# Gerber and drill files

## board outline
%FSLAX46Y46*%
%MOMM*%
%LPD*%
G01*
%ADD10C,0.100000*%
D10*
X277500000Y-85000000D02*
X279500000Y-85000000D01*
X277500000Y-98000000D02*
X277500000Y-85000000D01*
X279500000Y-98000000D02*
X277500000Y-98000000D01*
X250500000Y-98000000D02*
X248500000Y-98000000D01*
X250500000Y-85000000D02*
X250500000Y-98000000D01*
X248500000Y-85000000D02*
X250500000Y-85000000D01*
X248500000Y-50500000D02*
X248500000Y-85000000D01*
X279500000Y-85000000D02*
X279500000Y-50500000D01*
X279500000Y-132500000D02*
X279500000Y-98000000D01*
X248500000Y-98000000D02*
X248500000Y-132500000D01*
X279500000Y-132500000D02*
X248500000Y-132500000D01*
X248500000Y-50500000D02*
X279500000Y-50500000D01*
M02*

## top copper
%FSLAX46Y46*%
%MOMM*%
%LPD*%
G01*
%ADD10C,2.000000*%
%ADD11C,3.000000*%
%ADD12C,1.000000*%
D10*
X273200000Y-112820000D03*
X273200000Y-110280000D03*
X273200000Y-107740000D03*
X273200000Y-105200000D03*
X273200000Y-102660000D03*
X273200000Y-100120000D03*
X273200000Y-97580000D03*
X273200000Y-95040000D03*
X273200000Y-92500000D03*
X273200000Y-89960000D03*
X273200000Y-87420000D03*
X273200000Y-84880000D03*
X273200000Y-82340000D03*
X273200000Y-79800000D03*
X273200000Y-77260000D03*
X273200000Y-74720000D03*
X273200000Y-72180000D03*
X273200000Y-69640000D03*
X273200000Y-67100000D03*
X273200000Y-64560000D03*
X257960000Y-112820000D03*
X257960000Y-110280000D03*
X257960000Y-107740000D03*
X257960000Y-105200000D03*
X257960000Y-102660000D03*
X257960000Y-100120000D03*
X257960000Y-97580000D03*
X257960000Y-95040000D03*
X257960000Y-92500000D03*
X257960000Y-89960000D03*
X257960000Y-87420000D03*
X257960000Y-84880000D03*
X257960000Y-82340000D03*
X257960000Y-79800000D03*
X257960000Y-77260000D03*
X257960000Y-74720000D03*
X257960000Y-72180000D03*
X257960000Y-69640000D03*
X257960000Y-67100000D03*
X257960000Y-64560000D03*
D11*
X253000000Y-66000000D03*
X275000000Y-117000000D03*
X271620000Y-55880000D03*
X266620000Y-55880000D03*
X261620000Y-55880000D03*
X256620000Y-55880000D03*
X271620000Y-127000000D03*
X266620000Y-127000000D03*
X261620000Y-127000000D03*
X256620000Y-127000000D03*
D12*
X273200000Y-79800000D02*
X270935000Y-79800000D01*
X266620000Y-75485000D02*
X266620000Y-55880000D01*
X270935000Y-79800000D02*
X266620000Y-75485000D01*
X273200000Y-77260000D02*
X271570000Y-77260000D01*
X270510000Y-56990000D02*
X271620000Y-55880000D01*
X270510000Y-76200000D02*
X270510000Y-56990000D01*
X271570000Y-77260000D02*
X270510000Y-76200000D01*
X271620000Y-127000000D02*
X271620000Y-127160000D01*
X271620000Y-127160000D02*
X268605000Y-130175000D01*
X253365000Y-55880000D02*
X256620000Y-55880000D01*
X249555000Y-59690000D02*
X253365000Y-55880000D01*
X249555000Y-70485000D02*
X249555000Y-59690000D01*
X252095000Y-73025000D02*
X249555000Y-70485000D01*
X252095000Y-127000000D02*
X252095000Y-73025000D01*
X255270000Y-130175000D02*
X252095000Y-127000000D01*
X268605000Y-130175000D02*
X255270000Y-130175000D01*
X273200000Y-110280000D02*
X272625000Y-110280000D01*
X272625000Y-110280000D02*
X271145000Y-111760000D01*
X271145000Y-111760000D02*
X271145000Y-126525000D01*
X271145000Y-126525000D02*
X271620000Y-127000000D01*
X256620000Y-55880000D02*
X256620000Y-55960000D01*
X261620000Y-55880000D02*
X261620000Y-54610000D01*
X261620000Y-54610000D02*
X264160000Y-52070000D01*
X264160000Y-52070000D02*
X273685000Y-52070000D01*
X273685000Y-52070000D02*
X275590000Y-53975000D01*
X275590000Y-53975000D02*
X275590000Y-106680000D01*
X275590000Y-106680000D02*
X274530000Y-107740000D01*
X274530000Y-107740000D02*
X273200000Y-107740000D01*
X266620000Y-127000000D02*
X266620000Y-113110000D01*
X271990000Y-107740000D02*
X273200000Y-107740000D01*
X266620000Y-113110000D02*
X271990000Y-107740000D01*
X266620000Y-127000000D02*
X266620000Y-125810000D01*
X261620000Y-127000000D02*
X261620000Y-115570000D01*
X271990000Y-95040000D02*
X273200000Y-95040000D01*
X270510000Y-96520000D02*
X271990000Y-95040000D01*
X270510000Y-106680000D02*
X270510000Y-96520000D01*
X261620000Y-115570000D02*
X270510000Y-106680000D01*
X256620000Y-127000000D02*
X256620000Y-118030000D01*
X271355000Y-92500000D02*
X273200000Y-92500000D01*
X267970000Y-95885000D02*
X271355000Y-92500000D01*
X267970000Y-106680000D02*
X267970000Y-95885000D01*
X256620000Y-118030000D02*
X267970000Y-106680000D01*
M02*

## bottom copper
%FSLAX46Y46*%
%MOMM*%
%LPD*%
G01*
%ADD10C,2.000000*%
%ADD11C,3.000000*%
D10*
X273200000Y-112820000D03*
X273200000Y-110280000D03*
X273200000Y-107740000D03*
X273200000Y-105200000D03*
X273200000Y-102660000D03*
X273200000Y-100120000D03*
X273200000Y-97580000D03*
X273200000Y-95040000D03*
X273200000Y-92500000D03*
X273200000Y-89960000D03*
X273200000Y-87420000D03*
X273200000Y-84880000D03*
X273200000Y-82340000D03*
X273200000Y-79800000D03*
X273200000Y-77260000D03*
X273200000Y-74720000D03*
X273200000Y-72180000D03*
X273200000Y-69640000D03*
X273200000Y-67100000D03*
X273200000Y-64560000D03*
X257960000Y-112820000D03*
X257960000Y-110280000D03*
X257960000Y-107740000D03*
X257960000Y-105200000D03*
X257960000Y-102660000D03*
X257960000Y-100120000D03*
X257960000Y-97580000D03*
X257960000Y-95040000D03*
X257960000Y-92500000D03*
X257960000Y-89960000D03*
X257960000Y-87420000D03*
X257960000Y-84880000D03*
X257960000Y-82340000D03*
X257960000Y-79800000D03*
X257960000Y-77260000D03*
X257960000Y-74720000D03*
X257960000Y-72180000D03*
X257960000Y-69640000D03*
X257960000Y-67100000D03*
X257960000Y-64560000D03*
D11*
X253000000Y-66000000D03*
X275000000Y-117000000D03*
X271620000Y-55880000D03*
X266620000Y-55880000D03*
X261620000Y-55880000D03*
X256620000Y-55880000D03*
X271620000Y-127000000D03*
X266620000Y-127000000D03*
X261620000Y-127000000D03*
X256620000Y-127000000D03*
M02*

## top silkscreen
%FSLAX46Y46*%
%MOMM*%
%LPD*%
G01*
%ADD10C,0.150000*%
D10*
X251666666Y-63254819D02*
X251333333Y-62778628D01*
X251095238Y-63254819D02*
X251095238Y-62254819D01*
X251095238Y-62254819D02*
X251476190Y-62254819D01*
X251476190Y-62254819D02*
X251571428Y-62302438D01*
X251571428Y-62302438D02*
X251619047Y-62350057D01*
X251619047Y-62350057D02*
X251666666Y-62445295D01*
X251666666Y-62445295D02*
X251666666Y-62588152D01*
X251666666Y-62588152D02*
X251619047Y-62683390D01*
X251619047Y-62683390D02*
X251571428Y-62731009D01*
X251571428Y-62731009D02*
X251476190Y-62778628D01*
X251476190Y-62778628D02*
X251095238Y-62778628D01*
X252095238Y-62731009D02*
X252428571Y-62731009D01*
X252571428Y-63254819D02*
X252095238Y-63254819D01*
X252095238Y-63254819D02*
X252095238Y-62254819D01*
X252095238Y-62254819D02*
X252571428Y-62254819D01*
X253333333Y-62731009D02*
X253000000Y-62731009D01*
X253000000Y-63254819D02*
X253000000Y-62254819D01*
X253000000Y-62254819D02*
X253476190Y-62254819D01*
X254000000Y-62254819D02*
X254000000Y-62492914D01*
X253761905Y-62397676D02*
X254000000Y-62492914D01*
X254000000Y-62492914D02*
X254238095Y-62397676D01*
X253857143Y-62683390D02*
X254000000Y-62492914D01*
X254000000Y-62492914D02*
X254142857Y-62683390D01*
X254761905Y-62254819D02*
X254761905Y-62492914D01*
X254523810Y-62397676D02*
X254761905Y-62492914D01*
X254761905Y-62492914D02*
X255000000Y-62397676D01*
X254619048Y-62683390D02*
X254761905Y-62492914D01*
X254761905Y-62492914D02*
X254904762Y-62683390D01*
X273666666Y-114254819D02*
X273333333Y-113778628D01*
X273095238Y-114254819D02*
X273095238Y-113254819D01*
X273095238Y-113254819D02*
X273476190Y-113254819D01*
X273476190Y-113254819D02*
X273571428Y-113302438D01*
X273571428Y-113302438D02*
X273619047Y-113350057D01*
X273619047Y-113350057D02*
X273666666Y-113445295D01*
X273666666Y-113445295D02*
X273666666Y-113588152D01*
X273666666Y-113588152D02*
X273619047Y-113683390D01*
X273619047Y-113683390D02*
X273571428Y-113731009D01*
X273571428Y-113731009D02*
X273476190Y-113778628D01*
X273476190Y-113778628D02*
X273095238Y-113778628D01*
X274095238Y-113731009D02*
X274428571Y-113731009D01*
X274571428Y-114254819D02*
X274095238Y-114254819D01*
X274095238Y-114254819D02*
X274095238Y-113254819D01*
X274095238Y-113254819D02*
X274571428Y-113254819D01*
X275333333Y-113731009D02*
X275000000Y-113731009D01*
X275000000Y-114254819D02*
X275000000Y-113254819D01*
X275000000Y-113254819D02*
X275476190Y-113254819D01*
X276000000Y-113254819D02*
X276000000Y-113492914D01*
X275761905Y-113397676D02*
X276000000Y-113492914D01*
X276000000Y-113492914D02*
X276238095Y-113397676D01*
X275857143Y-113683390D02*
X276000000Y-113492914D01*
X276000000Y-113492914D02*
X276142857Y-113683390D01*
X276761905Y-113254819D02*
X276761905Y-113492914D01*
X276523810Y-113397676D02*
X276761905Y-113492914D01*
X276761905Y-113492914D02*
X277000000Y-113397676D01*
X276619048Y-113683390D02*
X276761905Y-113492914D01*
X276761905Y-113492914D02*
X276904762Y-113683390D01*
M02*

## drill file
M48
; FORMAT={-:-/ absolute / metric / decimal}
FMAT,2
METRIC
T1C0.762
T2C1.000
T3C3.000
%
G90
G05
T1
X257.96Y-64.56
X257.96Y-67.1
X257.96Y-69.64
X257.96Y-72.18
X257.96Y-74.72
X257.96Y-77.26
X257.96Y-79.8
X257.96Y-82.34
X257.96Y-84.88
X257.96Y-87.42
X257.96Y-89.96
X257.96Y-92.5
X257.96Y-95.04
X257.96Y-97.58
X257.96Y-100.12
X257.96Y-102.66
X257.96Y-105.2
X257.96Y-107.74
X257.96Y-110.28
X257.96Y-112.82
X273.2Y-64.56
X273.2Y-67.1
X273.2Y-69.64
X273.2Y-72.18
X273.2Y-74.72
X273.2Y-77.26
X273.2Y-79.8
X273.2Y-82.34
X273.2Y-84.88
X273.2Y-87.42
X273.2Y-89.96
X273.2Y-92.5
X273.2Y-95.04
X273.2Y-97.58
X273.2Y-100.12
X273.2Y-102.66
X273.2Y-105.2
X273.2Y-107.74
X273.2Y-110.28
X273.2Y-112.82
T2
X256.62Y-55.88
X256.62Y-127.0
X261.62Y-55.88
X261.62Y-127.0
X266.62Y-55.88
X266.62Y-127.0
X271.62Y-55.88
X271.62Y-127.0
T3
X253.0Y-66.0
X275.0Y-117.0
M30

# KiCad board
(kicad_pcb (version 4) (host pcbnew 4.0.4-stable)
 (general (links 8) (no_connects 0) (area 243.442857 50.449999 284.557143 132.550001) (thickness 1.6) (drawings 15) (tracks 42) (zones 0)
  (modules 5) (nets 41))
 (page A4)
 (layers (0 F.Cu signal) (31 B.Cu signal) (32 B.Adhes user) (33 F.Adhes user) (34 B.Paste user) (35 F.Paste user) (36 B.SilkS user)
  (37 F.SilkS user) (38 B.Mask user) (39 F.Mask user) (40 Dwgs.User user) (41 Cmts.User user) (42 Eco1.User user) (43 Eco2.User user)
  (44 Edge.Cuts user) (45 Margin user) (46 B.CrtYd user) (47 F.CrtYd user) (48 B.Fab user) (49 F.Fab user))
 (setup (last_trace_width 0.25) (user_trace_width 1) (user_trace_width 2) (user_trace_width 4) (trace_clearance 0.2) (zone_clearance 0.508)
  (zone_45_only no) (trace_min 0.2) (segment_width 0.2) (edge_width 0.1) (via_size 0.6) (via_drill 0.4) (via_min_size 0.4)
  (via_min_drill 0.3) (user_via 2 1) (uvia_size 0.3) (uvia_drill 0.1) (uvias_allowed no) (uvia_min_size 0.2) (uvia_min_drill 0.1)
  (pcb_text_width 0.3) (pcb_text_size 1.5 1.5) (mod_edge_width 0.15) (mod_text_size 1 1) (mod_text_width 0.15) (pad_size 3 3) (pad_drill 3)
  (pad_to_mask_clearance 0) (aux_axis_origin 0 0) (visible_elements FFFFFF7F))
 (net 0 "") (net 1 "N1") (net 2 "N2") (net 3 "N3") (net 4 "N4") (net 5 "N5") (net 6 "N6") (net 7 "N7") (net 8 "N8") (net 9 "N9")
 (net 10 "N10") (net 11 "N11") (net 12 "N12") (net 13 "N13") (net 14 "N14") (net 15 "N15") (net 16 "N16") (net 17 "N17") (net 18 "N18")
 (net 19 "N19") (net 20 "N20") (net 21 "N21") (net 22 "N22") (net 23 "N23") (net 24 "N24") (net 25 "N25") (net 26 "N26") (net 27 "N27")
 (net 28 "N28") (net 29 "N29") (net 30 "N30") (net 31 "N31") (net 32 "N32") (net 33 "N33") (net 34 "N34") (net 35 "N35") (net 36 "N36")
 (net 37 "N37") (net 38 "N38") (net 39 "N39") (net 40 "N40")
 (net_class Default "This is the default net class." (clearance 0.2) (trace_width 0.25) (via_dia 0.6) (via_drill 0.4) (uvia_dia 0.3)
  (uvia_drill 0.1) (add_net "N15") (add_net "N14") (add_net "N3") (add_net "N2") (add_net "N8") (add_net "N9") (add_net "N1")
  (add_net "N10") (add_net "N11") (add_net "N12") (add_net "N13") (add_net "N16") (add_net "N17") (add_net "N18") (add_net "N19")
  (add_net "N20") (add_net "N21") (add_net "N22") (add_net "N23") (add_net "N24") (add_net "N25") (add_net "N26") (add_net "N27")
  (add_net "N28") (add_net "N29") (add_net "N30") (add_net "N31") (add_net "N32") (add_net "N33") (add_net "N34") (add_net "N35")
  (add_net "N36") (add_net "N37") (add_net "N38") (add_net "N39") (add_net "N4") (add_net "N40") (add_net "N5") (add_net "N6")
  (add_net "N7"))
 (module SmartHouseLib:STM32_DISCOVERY (layer B.Cu) (at 260.5 92.5)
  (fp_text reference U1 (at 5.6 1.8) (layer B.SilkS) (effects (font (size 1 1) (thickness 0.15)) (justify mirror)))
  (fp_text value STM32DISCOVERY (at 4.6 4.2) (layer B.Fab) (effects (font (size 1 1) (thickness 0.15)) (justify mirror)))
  (pad 1 thru_hole circle (at 12.7 20.32) (size 2 2) (drill 0.762) (layers *.Cu *.Mask) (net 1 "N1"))
  (pad 2 thru_hole circle (at 12.7 17.78) (size 2 2) (drill 0.762) (layers *.Cu *.Mask) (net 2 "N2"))
  (pad 3 thru_hole circle (at 12.7 15.24) (size 2 2) (drill 0.762) (layers *.Cu *.Mask) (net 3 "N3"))
  (pad 4 thru_hole circle (at 12.7 12.7) (size 2 2) (drill 0.762) (layers *.Cu *.Mask) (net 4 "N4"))
  (pad 5 thru_hole circle (at 12.7 10.16) (size 2 2) (drill 0.762) (layers *.Cu *.Mask) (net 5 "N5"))
  (pad 6 thru_hole circle (at 12.7 7.62) (size 2 2) (drill 0.762) (layers *.Cu *.Mask) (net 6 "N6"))
  (pad 7 thru_hole circle (at 12.7 5.08) (size 2 2) (drill 0.762) (layers *.Cu *.Mask) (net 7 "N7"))
  (pad 8 thru_hole circle (at 12.7 2.54) (size 2 2) (drill 0.762) (layers *.Cu *.Mask) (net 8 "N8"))
  (pad 9 thru_hole circle (at 12.7 0) (size 2 2) (drill 0.762) (layers *.Cu *.Mask) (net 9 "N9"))
  (pad 10 thru_hole circle (at 12.7 -2.54) (size 2 2) (drill 0.762) (layers *.Cu *.Mask) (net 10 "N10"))
  (pad 11 thru_hole circle (at 12.7 -5.08) (size 2 2) (drill 0.762) (layers *.Cu *.Mask) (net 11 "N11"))
  (pad 12 thru_hole circle (at 12.7 -7.62) (size 2 2) (drill 0.762) (layers *.Cu *.Mask) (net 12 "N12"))
  (pad 13 thru_hole circle (at 12.7 -10.16) (size 2 2) (drill 0.762) (layers *.Cu *.Mask) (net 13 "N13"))
  (pad 14 thru_hole circle (at 12.7 -12.7) (size 2 2) (drill 0.762) (layers *.Cu *.Mask) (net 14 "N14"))
  (pad 15 thru_hole circle (at 12.7 -15.24) (size 2 2) (drill 0.762) (layers *.Cu *.Mask) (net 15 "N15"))
  (pad 16 thru_hole circle (at 12.7 -17.78) (size 2 2) (drill 0.762) (layers *.Cu *.Mask) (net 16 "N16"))
  (pad 17 thru_hole circle (at 12.7 -20.32) (size 2 2) (drill 0.762) (layers *.Cu *.Mask) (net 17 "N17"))
  (pad 18 thru_hole circle (at 12.7 -22.86) (size 2 2) (drill 0.762) (layers *.Cu *.Mask) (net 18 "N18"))
  (pad 19 thru_hole circle (at 12.7 -25.4) (size 2 2) (drill 0.762) (layers *.Cu *.Mask) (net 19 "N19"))
  (pad 20 thru_hole circle (at 12.7 -27.94) (size 2 2) (drill 0.762) (layers *.Cu *.Mask) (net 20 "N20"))
  (pad 21 thru_hole circle (at -2.54 20.32) (size 2 2) (drill 0.762) (layers *.Cu *.Mask) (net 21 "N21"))
  (pad 22 thru_hole circle (at -2.54 17.78) (size 2 2) (drill 0.762) (layers *.Cu *.Mask) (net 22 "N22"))
  (pad 23 thru_hole circle (at -2.54 15.24) (size 2 2) (drill 0.762) (layers *.Cu *.Mask) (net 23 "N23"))
  (pad 24 thru_hole circle (at -2.54 12.7) (size 2 2) (drill 0.762) (layers *.Cu *.Mask) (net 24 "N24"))
  (pad 25 thru_hole circle (at -2.54 10.16) (size 2 2) (drill 0.762) (layers *.Cu *.Mask) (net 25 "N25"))
  (pad 26 thru_hole circle (at -2.54 7.62) (size 2 2) (drill 0.762) (layers *.Cu *.Mask) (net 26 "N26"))
  (pad 27 thru_hole circle (at -2.54 5.08) (size 2 2) (drill 0.762) (layers *.Cu *.Mask) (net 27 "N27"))
  (pad 28 thru_hole circle (at -2.54 2.54) (size 2 2) (drill 0.762) (layers *.Cu *.Mask) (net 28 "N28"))
  (pad 29 thru_hole circle (at -2.54 0) (size 2 2) (drill 0.762) (layers *.Cu *.Mask) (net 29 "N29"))
  (pad 30 thru_hole circle (at -2.54 -2.54) (size 2 2) (drill 0.762) (layers *.Cu *.Mask) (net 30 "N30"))
  (pad 31 thru_hole circle (at -2.54 -5.08) (size 2 2) (drill 0.762) (layers *.Cu *.Mask) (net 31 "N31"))
  (pad 32 thru_hole circle (at -2.54 -7.62) (size 2 2) (drill 0.762) (layers *.Cu *.Mask) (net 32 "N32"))
  (pad 33 thru_hole circle (at -2.54 -10.16) (size 2 2) (drill 0.762) (layers *.Cu *.Mask) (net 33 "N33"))
  (pad 34 thru_hole circle (at -2.54 -12.7) (size 2 2) (drill 0.762) (layers *.Cu *.Mask) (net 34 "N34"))
  (pad 35 thru_hole circle (at -2.54 -15.24) (size 2 2) (drill 0.762) (layers *.Cu *.Mask) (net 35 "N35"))
  (pad 36 thru_hole circle (at -2.54 -17.78) (size 2 2) (drill 0.762) (layers *.Cu *.Mask) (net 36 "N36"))
  (pad 37 thru_hole circle (at -2.54 -20.32) (size 2 2) (drill 0.762) (layers *.Cu *.Mask) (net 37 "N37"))
  (pad 38 thru_hole circle (at -2.54 -22.86) (size 2 2) (drill 0.762) (layers *.Cu *.Mask) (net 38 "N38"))
  (pad 39 thru_hole circle (at -2.54 -25.4) (size 2 2) (drill 0.762) (layers *.Cu *.Mask) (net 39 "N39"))
  (pad 40 thru_hole circle (at -2.54 -27.94) (size 2 2) (drill 0.762) (layers *.Cu *.Mask) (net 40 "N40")))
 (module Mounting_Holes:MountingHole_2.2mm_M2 (layer F.Cu) (at 253 66)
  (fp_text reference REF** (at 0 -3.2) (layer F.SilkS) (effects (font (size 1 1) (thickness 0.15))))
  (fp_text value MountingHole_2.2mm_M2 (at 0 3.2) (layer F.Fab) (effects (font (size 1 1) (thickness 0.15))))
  (pad 1 thru_hole circle (at 0 0) (size 3 3) (drill 3) (layers *.Cu *.Mask)))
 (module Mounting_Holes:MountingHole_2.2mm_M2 (layer F.Cu) (at 275 117)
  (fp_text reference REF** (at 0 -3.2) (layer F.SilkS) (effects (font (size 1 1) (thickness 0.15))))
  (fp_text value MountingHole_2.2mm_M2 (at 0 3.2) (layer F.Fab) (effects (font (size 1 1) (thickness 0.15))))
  (pad 1 thru_hole circle (at 0 0) (size 3 3) (drill 3) (layers *.Cu *.Mask)))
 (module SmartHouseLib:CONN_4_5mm (layer B.Cu) (at 261.62 55.88 180)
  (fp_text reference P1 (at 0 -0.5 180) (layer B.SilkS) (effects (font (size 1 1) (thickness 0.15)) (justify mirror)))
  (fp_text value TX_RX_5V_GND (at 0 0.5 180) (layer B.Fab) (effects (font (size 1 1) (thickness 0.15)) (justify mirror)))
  (pad 1 thru_hole circle (at -10 0 180) (size 3 3) (drill 1) (layers *.Cu *.Mask) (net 15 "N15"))
  (pad 2 thru_hole circle (at -5 0 180) (size 3 3) (drill 1) (layers *.Cu *.Mask) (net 14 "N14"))
  (pad 3 thru_hole circle (at 0 0 180) (size 3 3) (drill 1) (layers *.Cu *.Mask) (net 3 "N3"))
  (pad 4 thru_hole circle (at 5 0 180) (size 3 3) (drill 1) (layers *.Cu *.Mask) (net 2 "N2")))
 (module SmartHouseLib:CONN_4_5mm (layer B.Cu) (at 261.62 127 180)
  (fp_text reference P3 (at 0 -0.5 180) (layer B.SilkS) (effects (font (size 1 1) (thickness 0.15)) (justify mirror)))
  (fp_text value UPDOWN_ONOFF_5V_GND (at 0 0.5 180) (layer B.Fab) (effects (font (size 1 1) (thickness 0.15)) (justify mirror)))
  (pad 1 thru_hole circle (at -10 0 180) (size 3 3) (drill 1) (layers *.Cu *.Mask) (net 2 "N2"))
  (pad 2 thru_hole circle (at -5 0 180) (size 3 3) (drill 1) (layers *.Cu *.Mask) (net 3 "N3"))
  (pad 3 thru_hole circle (at 0 0 180) (size 3 3) (drill 1) (layers *.Cu *.Mask) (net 8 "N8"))
  (pad 4 thru_hole circle (at 5 0 180) (size 3 3) (drill 1) (layers *.Cu *.Mask) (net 9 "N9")))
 (gr_line (start 277.5 85) (end 279.5 85) (angle 90) (layer Edge.Cuts) (width 0.1))
 (gr_line (start 277.5 98) (end 277.5 85) (angle 90) (layer Edge.Cuts) (width 0.1))
 (gr_line (start 279.5 98) (end 277.5 98) (angle 90) (layer Edge.Cuts) (width 0.1))
 (gr_line (start 250.5 98) (end 248.5 98) (angle 90) (layer Edge.Cuts) (width 0.1))
 (gr_line (start 250.5 85) (end 250.5 98) (angle 90) (layer Edge.Cuts) (width 0.1))
 (gr_line (start 248.5 85) (end 250.5 85) (angle 90) (layer Edge.Cuts) (width 0.1))
 (gr_line (start 248.5 50.5) (end 248.5 85) (angle 90) (layer Edge.Cuts) (width 0.1))
 (gr_line (start 279.5 85) (end 279.5 50.5) (angle 90) (layer Edge.Cuts) (width 0.1))
 (gr_line (start 279.5 132.5) (end 279.5 98) (angle 90) (layer Edge.Cuts) (width 0.1))
 (gr_line (start 248.5 98) (end 248.5 132.5) (angle 90) (layer Edge.Cuts) (width 0.1))
 (gr_line (start 279.5 132.5) (end 248.5 132.5) (angle 90) (layer Edge.Cuts) (width 0.1))
 (gr_line (start 248.5 50.5) (end 279.5 50.5) (angle 90) (layer Edge.Cuts) (width 0.1))
 (segment (start 273.2 79.8) (end 270.935 79.8) (width 1) (layer F.Cu) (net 14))
 (segment (start 266.62 75.485) (end 266.62 55.88) (width 1) (layer F.Cu) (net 14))
 (segment (start 270.935 79.8) (end 266.62 75.485) (width 1) (layer F.Cu) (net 14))
 (segment (start 273.2 77.26) (end 271.57 77.26) (width 1) (layer F.Cu) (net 15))
 (segment (start 270.51 56.99) (end 271.62 55.88) (width 1) (layer F.Cu) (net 15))
 (segment (start 270.51 76.2) (end 270.51 56.99) (width 1) (layer F.Cu) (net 15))
 (segment (start 271.57 77.26) (end 270.51 76.2) (width 1) (layer F.Cu) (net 15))
 (segment (start 271.62 127) (end 271.62 127.16) (width 1) (layer F.Cu) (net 2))
 (segment (start 271.62 127.16) (end 268.605 130.175) (width 1) (layer F.Cu) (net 2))
 (segment (start 253.365 55.88) (end 256.62 55.88) (width 1) (layer F.Cu) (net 2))
 (segment (start 249.555 59.69) (end 253.365 55.88) (width 1) (layer F.Cu) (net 2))
 (segment (start 249.555 70.485) (end 249.555 59.69) (width 1) (layer F.Cu) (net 2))
 (segment (start 252.095 73.025) (end 249.555 70.485) (width 1) (layer F.Cu) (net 2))
 (segment (start 252.095 127) (end 252.095 73.025) (width 1) (layer F.Cu) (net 2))
 (segment (start 255.27 130.175) (end 252.095 127) (width 1) (layer F.Cu) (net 2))
 (segment (start 268.605 130.175) (end 255.27 130.175) (width 1) (layer F.Cu) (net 2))
 (segment (start 273.2 110.28) (end 272.625 110.28) (width 1) (layer F.Cu) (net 2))
 (segment (start 272.625 110.28) (end 271.145 111.76) (width 1) (layer F.Cu) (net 2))
 (segment (start 271.145 111.76) (end 271.145 126.525) (width 1) (layer F.Cu) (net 2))
 (segment (start 271.145 126.525) (end 271.62 127) (width 1) (layer F.Cu) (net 2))
 (segment (start 256.62 55.88) (end 256.62 55.96) (width 1) (layer F.Cu) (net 2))
 (segment (start 261.62 55.88) (end 261.62 54.61) (width 1) (layer F.Cu) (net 3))
 (segment (start 261.62 54.61) (end 264.16 52.07) (width 1) (layer F.Cu) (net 3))
 (segment (start 264.16 52.07) (end 273.685 52.07) (width 1) (layer F.Cu) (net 3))
 (segment (start 273.685 52.07) (end 275.59 53.975) (width 1) (layer F.Cu) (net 3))
 (segment (start 275.59 53.975) (end 275.59 106.68) (width 1) (layer F.Cu) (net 3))
 (segment (start 275.59 106.68) (end 274.53 107.74) (width 1) (layer F.Cu) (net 3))
 (segment (start 274.53 107.74) (end 273.2 107.74) (width 1) (layer F.Cu) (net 3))
 (segment (start 266.62 127) (end 266.62 113.11) (width 1) (layer F.Cu) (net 3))
 (segment (start 271.99 107.74) (end 273.2 107.74) (width 1) (layer F.Cu) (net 3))
 (segment (start 266.62 113.11) (end 271.99 107.74) (width 1) (layer F.Cu) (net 3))
 (segment (start 266.62 127) (end 266.62 125.81) (width 1) (layer F.Cu) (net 3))
 (segment (start 261.62 127) (end 261.62 115.57) (width 1) (layer F.Cu) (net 8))
 (segment (start 271.99 95.04) (end 273.2 95.04) (width 1) (layer F.Cu) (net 8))
 (segment (start 270.51 96.52) (end 271.99 95.04) (width 1) (layer F.Cu) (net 8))
 (segment (start 270.51 106.68) (end 270.51 96.52) (width 1) (layer F.Cu) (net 8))
 (segment (start 261.62 115.57) (end 270.51 106.68) (width 1) (layer F.Cu) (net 8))
 (segment (start 256.62 127) (end 256.62 118.03) (width 1) (layer F.Cu) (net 9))
 (segment (start 271.355 92.5) (end 273.2 92.5) (width 1) (layer F.Cu) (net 9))
 (segment (start 267.97 95.885) (end 271.355 92.5) (width 1) (layer F.Cu) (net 9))
 (segment (start 267.97 106.68) (end 267.97 95.885) (width 1) (layer F.Cu) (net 9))
 (segment (start 256.62 118.03) (end 267.97 106.68) (width 1) (layer F.Cu) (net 9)))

